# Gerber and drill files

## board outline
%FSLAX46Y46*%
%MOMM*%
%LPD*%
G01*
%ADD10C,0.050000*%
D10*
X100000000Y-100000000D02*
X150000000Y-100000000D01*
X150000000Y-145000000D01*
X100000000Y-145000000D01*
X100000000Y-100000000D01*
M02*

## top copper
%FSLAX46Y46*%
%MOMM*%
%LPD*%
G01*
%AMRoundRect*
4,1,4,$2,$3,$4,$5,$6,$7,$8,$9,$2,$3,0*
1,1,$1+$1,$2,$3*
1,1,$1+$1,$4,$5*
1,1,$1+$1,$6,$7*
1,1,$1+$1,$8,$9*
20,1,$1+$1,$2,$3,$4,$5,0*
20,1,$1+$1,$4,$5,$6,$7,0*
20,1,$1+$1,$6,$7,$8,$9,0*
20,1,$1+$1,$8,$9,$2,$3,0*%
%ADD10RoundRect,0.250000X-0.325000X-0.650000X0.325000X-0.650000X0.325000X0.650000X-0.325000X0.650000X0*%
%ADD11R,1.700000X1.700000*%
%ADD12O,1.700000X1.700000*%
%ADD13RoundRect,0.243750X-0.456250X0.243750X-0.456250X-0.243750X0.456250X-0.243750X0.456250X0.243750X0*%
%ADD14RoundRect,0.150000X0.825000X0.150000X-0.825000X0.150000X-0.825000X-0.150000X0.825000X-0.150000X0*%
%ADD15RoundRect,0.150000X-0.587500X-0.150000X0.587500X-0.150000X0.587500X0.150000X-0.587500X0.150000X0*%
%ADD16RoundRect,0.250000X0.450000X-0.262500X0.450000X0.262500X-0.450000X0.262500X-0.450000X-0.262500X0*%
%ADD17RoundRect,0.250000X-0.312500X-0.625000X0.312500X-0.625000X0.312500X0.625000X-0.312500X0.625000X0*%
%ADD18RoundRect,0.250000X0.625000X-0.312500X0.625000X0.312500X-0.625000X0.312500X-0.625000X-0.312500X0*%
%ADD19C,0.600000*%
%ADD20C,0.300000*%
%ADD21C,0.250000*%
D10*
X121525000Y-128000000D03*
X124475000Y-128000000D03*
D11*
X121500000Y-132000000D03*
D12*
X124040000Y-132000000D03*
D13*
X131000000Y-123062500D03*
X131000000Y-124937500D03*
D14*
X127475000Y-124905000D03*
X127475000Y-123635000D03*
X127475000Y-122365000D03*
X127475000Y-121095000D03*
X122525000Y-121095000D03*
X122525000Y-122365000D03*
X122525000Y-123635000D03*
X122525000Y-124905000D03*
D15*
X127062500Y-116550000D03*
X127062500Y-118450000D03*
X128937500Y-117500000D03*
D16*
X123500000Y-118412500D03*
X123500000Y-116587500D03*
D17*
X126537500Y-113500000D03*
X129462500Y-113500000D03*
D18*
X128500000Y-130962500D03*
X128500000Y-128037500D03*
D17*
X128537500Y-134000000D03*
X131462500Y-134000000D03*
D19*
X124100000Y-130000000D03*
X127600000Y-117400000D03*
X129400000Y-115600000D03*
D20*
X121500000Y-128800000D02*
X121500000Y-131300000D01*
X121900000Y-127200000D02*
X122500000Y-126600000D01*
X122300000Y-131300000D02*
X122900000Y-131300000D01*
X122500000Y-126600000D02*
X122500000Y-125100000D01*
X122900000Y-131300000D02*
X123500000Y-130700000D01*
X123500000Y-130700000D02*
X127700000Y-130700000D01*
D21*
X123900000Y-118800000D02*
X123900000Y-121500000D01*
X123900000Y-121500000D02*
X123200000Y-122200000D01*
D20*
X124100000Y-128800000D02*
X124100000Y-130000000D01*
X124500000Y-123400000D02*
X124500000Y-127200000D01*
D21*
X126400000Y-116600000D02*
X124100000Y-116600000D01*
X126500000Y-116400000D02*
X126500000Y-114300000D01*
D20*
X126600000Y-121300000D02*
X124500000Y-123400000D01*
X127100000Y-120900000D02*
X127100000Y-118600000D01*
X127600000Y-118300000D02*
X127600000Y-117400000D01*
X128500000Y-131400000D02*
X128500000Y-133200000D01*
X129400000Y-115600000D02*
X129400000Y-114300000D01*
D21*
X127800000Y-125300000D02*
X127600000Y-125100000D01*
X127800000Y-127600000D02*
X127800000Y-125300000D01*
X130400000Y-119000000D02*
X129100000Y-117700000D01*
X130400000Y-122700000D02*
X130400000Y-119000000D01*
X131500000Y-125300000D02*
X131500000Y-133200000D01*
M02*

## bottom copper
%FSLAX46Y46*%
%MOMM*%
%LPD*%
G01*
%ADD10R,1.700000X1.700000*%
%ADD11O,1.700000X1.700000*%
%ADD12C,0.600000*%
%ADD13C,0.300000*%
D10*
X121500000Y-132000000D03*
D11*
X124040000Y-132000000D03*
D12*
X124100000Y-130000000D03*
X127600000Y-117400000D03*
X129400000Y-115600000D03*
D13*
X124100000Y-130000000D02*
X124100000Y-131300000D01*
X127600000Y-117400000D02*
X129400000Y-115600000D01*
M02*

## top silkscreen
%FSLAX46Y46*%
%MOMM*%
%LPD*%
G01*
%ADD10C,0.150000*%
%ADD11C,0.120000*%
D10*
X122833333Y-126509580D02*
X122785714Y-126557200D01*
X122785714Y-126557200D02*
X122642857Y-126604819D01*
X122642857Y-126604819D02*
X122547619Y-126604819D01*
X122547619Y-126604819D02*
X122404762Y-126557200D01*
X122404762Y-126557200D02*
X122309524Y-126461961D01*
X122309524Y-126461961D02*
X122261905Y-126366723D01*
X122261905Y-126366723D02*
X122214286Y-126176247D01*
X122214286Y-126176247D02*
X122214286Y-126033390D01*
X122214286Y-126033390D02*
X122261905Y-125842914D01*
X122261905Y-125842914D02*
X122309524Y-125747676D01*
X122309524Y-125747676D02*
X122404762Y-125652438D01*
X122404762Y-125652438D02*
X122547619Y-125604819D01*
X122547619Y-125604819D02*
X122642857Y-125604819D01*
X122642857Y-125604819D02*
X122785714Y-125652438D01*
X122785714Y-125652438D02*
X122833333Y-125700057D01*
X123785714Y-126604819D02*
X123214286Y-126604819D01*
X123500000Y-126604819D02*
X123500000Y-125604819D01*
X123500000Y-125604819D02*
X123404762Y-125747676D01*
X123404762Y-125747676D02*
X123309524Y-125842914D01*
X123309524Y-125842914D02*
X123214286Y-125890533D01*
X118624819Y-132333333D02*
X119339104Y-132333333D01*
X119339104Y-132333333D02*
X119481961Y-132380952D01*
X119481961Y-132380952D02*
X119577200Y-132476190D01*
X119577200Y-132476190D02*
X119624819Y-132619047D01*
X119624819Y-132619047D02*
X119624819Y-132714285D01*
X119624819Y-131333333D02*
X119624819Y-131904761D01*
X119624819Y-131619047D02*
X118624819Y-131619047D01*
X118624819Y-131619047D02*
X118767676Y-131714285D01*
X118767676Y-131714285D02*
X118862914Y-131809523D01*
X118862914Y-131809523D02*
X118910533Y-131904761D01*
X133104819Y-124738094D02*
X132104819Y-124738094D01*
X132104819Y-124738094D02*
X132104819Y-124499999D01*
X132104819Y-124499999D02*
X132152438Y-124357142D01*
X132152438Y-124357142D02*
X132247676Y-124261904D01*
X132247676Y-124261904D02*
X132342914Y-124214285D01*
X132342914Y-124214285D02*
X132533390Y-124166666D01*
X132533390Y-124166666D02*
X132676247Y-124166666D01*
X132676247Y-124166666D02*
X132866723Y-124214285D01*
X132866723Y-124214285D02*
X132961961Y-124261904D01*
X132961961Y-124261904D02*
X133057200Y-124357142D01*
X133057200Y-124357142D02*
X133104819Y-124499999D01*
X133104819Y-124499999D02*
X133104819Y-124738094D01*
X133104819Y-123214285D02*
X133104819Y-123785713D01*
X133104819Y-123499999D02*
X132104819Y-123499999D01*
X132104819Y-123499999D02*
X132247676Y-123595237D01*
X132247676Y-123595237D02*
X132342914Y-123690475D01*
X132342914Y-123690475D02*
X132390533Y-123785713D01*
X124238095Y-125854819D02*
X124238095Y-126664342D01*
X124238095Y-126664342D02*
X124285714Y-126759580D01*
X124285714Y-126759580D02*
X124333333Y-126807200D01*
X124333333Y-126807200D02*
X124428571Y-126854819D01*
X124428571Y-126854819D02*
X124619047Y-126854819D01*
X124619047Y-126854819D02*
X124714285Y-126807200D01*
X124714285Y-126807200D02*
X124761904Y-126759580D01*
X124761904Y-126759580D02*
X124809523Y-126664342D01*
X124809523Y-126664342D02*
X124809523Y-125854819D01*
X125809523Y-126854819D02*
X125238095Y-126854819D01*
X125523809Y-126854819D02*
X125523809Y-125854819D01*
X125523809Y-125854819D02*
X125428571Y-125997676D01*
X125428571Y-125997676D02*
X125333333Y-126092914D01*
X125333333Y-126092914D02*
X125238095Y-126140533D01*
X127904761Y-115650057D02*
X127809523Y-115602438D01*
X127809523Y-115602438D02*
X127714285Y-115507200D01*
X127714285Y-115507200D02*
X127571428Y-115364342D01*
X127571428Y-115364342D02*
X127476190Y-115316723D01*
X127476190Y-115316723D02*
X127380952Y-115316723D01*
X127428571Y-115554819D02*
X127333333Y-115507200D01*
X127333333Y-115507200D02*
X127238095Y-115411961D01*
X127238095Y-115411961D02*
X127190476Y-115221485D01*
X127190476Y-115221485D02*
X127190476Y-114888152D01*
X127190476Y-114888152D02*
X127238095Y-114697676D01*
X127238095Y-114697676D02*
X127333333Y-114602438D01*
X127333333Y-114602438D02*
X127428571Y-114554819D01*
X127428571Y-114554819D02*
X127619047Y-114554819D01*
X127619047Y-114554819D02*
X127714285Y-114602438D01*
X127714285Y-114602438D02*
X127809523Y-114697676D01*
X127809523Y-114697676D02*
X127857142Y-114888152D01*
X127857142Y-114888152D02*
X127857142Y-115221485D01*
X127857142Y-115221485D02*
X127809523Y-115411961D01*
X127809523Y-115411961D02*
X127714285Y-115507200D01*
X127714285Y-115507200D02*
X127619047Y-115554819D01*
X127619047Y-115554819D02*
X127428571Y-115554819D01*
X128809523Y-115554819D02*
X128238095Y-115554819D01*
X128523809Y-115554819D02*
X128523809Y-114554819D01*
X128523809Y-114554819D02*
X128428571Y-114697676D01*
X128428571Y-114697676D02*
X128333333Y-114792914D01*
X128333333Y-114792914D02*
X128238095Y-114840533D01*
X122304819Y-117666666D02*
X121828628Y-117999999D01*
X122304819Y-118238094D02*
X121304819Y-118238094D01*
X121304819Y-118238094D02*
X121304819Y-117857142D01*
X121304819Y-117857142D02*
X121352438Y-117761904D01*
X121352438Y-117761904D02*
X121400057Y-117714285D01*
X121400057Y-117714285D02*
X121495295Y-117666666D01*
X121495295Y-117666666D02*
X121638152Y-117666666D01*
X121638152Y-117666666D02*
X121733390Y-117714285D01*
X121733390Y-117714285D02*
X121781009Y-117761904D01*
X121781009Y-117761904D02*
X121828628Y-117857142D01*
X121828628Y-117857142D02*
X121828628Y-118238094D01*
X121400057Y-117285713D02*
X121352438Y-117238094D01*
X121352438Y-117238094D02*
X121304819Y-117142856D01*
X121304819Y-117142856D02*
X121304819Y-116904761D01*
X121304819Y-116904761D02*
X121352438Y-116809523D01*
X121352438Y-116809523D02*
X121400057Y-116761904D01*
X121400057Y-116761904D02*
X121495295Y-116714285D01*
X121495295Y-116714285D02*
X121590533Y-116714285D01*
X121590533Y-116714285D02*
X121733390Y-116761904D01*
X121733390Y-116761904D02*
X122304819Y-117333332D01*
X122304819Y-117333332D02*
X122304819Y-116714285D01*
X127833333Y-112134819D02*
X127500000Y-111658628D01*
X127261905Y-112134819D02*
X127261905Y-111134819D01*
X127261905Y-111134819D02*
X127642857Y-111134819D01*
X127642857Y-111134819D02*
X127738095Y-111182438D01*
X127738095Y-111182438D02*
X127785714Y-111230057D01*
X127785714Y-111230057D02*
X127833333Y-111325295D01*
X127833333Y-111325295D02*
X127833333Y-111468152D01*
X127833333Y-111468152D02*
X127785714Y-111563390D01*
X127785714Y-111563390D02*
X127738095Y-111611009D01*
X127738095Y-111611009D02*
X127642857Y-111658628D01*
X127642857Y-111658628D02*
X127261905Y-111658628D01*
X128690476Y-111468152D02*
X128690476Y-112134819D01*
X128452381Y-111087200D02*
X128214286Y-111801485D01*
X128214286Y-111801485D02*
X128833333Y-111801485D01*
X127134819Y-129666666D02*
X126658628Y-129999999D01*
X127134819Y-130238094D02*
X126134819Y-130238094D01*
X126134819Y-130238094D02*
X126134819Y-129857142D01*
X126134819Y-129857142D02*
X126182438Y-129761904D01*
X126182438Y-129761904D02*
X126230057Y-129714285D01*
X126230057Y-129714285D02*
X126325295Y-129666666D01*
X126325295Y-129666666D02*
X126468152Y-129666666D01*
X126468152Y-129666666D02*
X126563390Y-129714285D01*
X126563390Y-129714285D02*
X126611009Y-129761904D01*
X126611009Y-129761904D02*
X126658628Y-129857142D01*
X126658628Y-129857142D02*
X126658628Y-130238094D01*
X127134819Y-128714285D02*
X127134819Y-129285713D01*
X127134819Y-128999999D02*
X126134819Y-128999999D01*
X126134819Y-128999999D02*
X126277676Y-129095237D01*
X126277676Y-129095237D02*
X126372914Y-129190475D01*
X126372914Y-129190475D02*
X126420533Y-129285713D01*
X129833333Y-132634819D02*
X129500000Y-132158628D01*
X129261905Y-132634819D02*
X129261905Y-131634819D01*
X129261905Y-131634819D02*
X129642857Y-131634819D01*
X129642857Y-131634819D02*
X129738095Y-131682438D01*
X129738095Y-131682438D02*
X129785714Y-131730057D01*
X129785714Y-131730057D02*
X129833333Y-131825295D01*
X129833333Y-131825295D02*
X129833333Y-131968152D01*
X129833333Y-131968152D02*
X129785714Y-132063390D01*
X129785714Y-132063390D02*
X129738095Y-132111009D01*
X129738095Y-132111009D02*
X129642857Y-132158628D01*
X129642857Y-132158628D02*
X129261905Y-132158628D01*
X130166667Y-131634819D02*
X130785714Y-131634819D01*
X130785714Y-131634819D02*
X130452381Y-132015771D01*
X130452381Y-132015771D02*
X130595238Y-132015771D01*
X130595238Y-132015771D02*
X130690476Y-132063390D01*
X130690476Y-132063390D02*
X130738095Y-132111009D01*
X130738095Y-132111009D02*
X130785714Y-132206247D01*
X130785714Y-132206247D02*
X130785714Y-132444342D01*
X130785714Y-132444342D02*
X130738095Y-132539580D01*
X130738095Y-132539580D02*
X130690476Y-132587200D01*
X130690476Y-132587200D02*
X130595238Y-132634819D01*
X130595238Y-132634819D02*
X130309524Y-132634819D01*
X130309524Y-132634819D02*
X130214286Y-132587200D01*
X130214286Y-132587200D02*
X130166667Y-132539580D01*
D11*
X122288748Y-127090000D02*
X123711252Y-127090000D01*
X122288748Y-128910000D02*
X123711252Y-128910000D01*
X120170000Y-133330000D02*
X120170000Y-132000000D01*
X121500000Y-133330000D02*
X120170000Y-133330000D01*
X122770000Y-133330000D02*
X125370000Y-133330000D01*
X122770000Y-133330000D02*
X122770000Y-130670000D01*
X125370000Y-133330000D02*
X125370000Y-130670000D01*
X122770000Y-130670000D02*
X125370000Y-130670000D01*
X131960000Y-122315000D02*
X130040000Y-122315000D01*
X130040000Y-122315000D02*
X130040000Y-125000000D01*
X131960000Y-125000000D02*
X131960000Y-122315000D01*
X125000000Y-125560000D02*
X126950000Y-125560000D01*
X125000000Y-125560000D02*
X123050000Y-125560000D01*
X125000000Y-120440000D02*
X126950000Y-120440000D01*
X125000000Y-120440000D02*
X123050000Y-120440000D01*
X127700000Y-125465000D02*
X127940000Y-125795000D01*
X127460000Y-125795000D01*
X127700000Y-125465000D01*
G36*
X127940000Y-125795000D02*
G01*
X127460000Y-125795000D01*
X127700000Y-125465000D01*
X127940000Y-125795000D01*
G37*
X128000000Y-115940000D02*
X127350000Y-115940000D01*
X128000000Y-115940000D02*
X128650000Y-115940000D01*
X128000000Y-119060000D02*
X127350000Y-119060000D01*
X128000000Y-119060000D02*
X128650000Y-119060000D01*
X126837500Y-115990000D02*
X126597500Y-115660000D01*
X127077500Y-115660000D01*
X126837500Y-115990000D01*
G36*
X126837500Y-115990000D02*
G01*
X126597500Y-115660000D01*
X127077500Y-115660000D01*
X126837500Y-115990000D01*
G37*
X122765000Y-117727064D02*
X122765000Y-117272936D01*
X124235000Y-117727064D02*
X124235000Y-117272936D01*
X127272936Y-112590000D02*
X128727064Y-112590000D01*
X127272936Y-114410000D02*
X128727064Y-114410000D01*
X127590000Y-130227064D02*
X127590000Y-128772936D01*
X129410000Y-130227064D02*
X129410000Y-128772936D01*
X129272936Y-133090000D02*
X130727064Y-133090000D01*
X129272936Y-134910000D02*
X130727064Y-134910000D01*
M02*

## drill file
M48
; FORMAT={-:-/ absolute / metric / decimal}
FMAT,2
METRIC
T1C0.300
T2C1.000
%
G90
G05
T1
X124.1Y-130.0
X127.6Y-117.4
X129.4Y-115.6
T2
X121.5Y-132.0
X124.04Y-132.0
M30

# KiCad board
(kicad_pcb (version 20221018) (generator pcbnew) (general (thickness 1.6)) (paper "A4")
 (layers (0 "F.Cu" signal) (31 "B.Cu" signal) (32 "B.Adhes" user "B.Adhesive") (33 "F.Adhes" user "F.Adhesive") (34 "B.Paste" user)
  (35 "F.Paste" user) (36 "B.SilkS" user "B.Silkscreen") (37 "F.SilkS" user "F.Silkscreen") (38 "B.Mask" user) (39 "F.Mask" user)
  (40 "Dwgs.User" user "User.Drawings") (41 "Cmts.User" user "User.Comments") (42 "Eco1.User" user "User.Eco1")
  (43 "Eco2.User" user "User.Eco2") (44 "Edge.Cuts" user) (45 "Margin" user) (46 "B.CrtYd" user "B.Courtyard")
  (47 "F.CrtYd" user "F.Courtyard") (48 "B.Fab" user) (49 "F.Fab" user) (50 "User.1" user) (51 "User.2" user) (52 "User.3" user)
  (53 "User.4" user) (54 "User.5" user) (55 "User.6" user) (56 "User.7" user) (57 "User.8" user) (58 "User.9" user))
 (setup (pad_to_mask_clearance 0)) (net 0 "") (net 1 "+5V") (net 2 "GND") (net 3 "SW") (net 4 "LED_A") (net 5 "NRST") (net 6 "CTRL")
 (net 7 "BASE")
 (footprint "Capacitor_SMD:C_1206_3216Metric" (layer "F.Cu") (at 123 128)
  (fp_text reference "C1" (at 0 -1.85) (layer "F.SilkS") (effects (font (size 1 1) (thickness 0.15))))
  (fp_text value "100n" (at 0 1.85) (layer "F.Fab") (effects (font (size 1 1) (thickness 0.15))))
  (fp_line (start -0.711252 -0.91) (end 0.711252 -0.91) (stroke (width 0.12) (type solid)) (layer "F.SilkS"))
  (fp_line (start -0.711252 0.91) (end 0.711252 0.91) (stroke (width 0.12) (type solid)) (layer "F.SilkS"))
  (pad "1" smd roundrect (at -1.475 0) (size 1.15 1.8) (layers "F.Cu" "F.Paste" "F.Mask") (roundrect_rratio 0.217391) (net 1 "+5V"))
  (pad "2" smd roundrect (at 1.475 0) (size 1.15 1.8) (layers "F.Cu" "F.Paste" "F.Mask") (roundrect_rratio 0.217391) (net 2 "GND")))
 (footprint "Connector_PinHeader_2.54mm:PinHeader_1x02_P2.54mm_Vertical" (layer "F.Cu") (at 121.5 132 90)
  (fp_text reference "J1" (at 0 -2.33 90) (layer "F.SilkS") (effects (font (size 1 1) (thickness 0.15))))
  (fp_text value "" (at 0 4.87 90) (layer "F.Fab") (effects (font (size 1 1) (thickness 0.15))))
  (fp_line (start -1.33 -1.33) (end 0 -1.33) (stroke (width 0.12) (type solid)) (layer "F.SilkS"))
  (fp_line (start -1.33 0) (end -1.33 -1.33) (stroke (width 0.12) (type solid)) (layer "F.SilkS"))
  (fp_line (start -1.33 1.27) (end -1.33 3.87) (stroke (width 0.12) (type solid)) (layer "F.SilkS"))
  (fp_line (start -1.33 1.27) (end 1.33 1.27) (stroke (width 0.12) (type solid)) (layer "F.SilkS"))
  (fp_line (start -1.33 3.87) (end 1.33 3.87) (stroke (width 0.12) (type solid)) (layer "F.SilkS"))
  (fp_line (start 1.33 1.27) (end 1.33 3.87) (stroke (width 0.12) (type solid)) (layer "F.SilkS"))
  (pad "1" thru_hole rect (at 0 0 90) (size 1.7 1.7) (drill 1) (layers "*.Cu" "*.Mask") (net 1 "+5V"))
  (pad "2" thru_hole oval (at 0 2.54 90) (size 1.7 1.7) (drill 1) (layers "*.Cu" "*.Mask") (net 2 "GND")))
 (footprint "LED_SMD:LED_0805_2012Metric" (layer "F.Cu") (at 131 124 -90)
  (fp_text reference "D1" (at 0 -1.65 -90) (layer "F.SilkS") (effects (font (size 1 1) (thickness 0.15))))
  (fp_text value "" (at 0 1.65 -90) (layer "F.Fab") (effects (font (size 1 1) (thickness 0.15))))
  (fp_line (start -1.685 -0.96) (end -1.685 0.96) (stroke (width 0.12) (type solid)) (layer "F.SilkS"))
  (fp_line (start -1.685 0.96) (end 1 0.96) (stroke (width 0.12) (type solid)) (layer "F.SilkS"))
  (fp_line (start 1 -0.96) (end -1.685 -0.96) (stroke (width 0.12) (type solid)) (layer "F.SilkS"))
  (pad "1" smd roundrect (at -0.9375 0 270) (size 0.975 1.4) (layers "F.Cu" "F.Paste" "F.Mask") (roundrect_rratio 0.25) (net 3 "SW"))
  (pad "2" smd roundrect (at 0.9375 0 270) (size 0.975 1.4) (layers "F.Cu" "F.Paste" "F.Mask") (roundrect_rratio 0.25) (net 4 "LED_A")))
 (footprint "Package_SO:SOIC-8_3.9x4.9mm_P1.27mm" (layer "F.Cu") (at 125 123 180)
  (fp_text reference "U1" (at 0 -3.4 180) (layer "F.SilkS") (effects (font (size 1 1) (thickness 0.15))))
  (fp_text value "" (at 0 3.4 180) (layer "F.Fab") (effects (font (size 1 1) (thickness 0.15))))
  (fp_line (start 0 -2.56) (end -1.95 -2.56) (stroke (width 0.12) (type solid)) (layer "F.SilkS"))
  (fp_line (start 0 -2.56) (end 1.95 -2.56) (stroke (width 0.12) (type solid)) (layer "F.SilkS"))
  (fp_line (start 0 2.56) (end -1.95 2.56) (stroke (width 0.12) (type solid)) (layer "F.SilkS"))
  (fp_line (start 0 2.56) (end 1.95 2.56) (stroke (width 0.12) (type solid)) (layer "F.SilkS"))
  (fp_poly
   (pts (xy -2.7 -2.465) (xy -2.94 -2.795) (xy -2.46 -2.795) (xy -2.7 -2.465)) (stroke (width 0.12) (type solid)) (fill solid)
   (layer "F.SilkS"))
  (pad "1" smd roundrect (at -2.475 -1.905 180) (size 1.95 0.6) (layers "F.Cu" "F.Paste" "F.Mask") (roundrect_rratio 0.25) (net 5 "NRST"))
  (pad "2" smd roundrect (at -2.475 -0.635 180) (size 1.95 0.6) (layers "F.Cu" "F.Paste" "F.Mask") (roundrect_rratio 0.25))
  (pad "3" smd roundrect (at -2.475 0.635 180) (size 1.95 0.6) (layers "F.Cu" "F.Paste" "F.Mask") (roundrect_rratio 0.25))
  (pad "4" smd roundrect (at -2.475 1.905 180) (size 1.95 0.6) (layers "F.Cu" "F.Paste" "F.Mask") (roundrect_rratio 0.25) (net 2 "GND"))
  (pad "5" smd roundrect (at 2.475 1.905 180) (size 1.95 0.6) (layers "F.Cu" "F.Paste" "F.Mask") (roundrect_rratio 0.25))
  (pad "6" smd roundrect (at 2.475 0.635 180) (size 1.95 0.6) (layers "F.Cu" "F.Paste" "F.Mask") (roundrect_rratio 0.25) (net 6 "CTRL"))
  (pad "7" smd roundrect (at 2.475 -0.635 180) (size 1.95 0.6) (layers "F.Cu" "F.Paste" "F.Mask") (roundrect_rratio 0.25))
  (pad "8" smd roundrect (at 2.475 -1.905 180) (size 1.95 0.6) (layers "F.Cu" "F.Paste" "F.Mask") (roundrect_rratio 0.25) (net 1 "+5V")))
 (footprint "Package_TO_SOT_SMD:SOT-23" (layer "F.Cu") (at 128 117.5)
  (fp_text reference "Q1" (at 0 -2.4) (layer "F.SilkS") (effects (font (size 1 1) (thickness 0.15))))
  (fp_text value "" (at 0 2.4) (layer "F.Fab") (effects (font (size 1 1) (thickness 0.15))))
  (fp_line (start 0 -1.56) (end -0.65 -1.56) (stroke (width 0.12) (type solid)) (layer "F.SilkS"))
  (fp_line (start 0 -1.56) (end 0.65 -1.56) (stroke (width 0.12) (type solid)) (layer "F.SilkS"))
  (fp_line (start 0 1.56) (end -0.65 1.56) (stroke (width 0.12) (type solid)) (layer "F.SilkS"))
  (fp_line (start 0 1.56) (end 0.65 1.56) (stroke (width 0.12) (type solid)) (layer "F.SilkS"))
  (fp_poly
   (pts (xy -1.1625 -1.51) (xy -1.4025 -1.84) (xy -0.9225 -1.84) (xy -1.1625 -1.51)) (stroke (width 0.12) (type solid)) (fill solid)
   (layer "F.SilkS"))
  (pad "1" smd roundrect (at -0.9375 -0.95) (size 1.475 0.6) (layers "F.Cu" "F.Paste" "F.Mask") (roundrect_rratio 0.25) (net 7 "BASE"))
  (pad "2" smd roundrect (at -0.9375 0.95) (size 1.475 0.6) (layers "F.Cu" "F.Paste" "F.Mask") (roundrect_rratio 0.25) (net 2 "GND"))
  (pad "3" smd roundrect (at 0.9375 0) (size 1.475 0.6) (layers "F.Cu" "F.Paste" "F.Mask") (roundrect_rratio 0.25) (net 3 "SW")))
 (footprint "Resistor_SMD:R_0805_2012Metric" (layer "F.Cu") (at 123.5 117.5 90)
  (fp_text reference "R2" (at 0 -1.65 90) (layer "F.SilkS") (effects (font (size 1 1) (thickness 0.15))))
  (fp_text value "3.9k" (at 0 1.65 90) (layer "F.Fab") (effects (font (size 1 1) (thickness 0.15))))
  (fp_line (start -0.227064 -0.735) (end 0.227064 -0.735) (stroke (width 0.12) (type solid)) (layer "F.SilkS"))
  (fp_line (start -0.227064 0.735) (end 0.227064 0.735) (stroke (width 0.12) (type solid)) (layer "F.SilkS"))
  (pad "1" smd roundrect (at -0.9125 0 90) (size 1.025 1.4) (layers "F.Cu" "F.Paste" "F.Mask") (roundrect_rratio 0.243902) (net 6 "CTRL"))
  (pad "2" smd roundrect (at 0.9125 0 90) (size 1.025 1.4) (layers "F.Cu" "F.Paste" "F.Mask") (roundrect_rratio 0.243902) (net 7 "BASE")))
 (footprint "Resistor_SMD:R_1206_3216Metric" (layer "F.Cu") (at 128 113.5)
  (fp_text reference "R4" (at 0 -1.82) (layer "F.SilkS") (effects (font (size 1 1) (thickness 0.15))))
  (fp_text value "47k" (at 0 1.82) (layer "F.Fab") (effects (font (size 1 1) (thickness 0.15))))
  (fp_line (start -0.727064 -0.91) (end 0.727064 -0.91) (stroke (width 0.12) (type solid)) (layer "F.SilkS"))
  (fp_line (start -0.727064 0.91) (end 0.727064 0.91) (stroke (width 0.12) (type solid)) (layer "F.SilkS"))
  (pad "1" smd roundrect (at -1.4625 0) (size 1.125 1.75) (layers "F.Cu" "F.Paste" "F.Mask") (roundrect_rratio 0.222222) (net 7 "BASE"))
  (pad "2" smd roundrect (at 1.4625 0) (size 1.125 1.75) (layers "F.Cu" "F.Paste" "F.Mask") (roundrect_rratio 0.222222) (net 2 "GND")))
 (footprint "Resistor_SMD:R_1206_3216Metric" (layer "F.Cu") (at 128.5 129.5 90)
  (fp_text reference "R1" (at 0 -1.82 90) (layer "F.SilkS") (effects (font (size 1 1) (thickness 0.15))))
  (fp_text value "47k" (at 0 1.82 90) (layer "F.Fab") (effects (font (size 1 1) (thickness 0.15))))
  (fp_line (start -0.727064 -0.91) (end 0.727064 -0.91) (stroke (width 0.12) (type solid)) (layer "F.SilkS"))
  (fp_line (start -0.727064 0.91) (end 0.727064 0.91) (stroke (width 0.12) (type solid)) (layer "F.SilkS"))
  (pad "1" smd roundrect (at -1.4625 0 90) (size 1.125 1.75) (layers "F.Cu" "F.Paste" "F.Mask") (roundrect_rratio 0.222222) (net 1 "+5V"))
  (pad "2" smd roundrect (at 1.4625 0 90) (size 1.125 1.75) (layers "F.Cu" "F.Paste" "F.Mask") (roundrect_rratio 0.222222) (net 5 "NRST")))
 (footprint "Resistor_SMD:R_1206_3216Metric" (layer "F.Cu") (at 130 134)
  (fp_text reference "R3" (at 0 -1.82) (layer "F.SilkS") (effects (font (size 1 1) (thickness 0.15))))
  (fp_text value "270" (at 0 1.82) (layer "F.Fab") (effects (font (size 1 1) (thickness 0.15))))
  (fp_line (start -0.727064 -0.91) (end 0.727064 -0.91) (stroke (width 0.12) (type solid)) (layer "F.SilkS"))
  (fp_line (start -0.727064 0.91) (end 0.727064 0.91) (stroke (width 0.12) (type solid)) (layer "F.SilkS"))
  (pad "1" smd roundrect (at -1.4625 0) (size 1.125 1.75) (layers "F.Cu" "F.Paste" "F.Mask") (roundrect_rratio 0.222222) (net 1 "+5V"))
  (pad "2" smd roundrect (at 1.4625 0) (size 1.125 1.75) (layers "F.Cu" "F.Paste" "F.Mask") (roundrect_rratio 0.222222) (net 4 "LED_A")))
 (gr_rect (start 100 100) (end 150 145) (stroke (width 0.05) (type default)) (fill none) (layer "Edge.Cuts"))
 (segment (start 121.5 128.8) (end 121.5 131.3) (width 0.3) (layer "F.Cu") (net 1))
 (segment (start 121.9 127.2) (end 122.5 126.6) (width 0.3) (layer "F.Cu") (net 1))
 (segment (start 122.3 131.3) (end 122.9 131.3) (width 0.3) (layer "F.Cu") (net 1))
 (segment (start 122.5 126.6) (end 122.5 125.1) (width 0.3) (layer "F.Cu") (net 1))
 (segment (start 122.9 131.3) (end 123.5 130.7) (width 0.3) (layer "F.Cu") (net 1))
 (segment (start 123.5 130.7) (end 127.7 130.7) (width 0.3) (layer "F.Cu") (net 1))
 (segment (start 123.9 118.8) (end 123.9 121.5) (width 0.25) (layer "F.Cu") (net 6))
 (segment (start 123.9 121.5) (end 123.2 122.2) (width 0.25) (layer "F.Cu") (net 6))
 (segment (start 124.1 128.8) (end 124.1 130) (width 0.3) (layer "F.Cu") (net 2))
 (segment (start 124.5 123.4) (end 124.5 127.2) (width 0.3) (layer "F.Cu") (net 2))
 (segment (start 126.4 116.6) (end 124.1 116.6) (width 0.25) (layer "F.Cu") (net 7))
 (segment (start 126.5 116.4) (end 126.5 114.3) (width 0.25) (layer "F.Cu") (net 7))
 (segment (start 126.6 121.3) (end 124.5 123.4) (width 0.3) (layer "F.Cu") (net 2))
 (segment (start 127.1 120.9) (end 127.1 118.6) (width 0.3) (layer "F.Cu") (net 2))
 (segment (start 127.6 118.3) (end 127.6 117.4) (width 0.3) (layer "F.Cu") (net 2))
 (segment (start 128.5 131.4) (end 128.5 133.2) (width 0.3) (layer "F.Cu") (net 1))
 (segment (start 129.4 115.6) (end 129.4 114.3) (width 0.3) (layer "F.Cu") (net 2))
 (via (at 124.1 130) (size 0.6) (drill 0.3) (layers "F.Cu" "B.Cu") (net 2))
 (via (at 127.6 117.4) (size 0.6) (drill 0.3) (layers "F.Cu" "B.Cu") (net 2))
 (via (at 129.4 115.6) (size 0.6) (drill 0.3) (layers "F.Cu" "B.Cu") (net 2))
 (segment (start 124.1 130) (end 124.1 131.3) (width 0.3) (layer "B.Cu") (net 2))
 (segment (start 127.6 117.4) (end 129.4 115.6) (width 0.3) (layer "B.Cu") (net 2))
 (segment (start 127.8 125.3) (end 127.6 125.1) (width 0.25) (layer "F.Cu") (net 5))
 (segment (start 127.8 127.6) (end 127.8 125.3) (width 0.25) (layer "F.Cu") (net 5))
 (segment (start 130.4 119) (end 129.1 117.7) (width 0.25) (layer "F.Cu") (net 3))
 (segment (start 130.4 122.7) (end 130.4 119) (width 0.25) (layer "F.Cu") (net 3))
 (segment (start 131.5 125.3) (end 131.5 133.2) (width 0.25) (layer "F.Cu") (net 4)))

